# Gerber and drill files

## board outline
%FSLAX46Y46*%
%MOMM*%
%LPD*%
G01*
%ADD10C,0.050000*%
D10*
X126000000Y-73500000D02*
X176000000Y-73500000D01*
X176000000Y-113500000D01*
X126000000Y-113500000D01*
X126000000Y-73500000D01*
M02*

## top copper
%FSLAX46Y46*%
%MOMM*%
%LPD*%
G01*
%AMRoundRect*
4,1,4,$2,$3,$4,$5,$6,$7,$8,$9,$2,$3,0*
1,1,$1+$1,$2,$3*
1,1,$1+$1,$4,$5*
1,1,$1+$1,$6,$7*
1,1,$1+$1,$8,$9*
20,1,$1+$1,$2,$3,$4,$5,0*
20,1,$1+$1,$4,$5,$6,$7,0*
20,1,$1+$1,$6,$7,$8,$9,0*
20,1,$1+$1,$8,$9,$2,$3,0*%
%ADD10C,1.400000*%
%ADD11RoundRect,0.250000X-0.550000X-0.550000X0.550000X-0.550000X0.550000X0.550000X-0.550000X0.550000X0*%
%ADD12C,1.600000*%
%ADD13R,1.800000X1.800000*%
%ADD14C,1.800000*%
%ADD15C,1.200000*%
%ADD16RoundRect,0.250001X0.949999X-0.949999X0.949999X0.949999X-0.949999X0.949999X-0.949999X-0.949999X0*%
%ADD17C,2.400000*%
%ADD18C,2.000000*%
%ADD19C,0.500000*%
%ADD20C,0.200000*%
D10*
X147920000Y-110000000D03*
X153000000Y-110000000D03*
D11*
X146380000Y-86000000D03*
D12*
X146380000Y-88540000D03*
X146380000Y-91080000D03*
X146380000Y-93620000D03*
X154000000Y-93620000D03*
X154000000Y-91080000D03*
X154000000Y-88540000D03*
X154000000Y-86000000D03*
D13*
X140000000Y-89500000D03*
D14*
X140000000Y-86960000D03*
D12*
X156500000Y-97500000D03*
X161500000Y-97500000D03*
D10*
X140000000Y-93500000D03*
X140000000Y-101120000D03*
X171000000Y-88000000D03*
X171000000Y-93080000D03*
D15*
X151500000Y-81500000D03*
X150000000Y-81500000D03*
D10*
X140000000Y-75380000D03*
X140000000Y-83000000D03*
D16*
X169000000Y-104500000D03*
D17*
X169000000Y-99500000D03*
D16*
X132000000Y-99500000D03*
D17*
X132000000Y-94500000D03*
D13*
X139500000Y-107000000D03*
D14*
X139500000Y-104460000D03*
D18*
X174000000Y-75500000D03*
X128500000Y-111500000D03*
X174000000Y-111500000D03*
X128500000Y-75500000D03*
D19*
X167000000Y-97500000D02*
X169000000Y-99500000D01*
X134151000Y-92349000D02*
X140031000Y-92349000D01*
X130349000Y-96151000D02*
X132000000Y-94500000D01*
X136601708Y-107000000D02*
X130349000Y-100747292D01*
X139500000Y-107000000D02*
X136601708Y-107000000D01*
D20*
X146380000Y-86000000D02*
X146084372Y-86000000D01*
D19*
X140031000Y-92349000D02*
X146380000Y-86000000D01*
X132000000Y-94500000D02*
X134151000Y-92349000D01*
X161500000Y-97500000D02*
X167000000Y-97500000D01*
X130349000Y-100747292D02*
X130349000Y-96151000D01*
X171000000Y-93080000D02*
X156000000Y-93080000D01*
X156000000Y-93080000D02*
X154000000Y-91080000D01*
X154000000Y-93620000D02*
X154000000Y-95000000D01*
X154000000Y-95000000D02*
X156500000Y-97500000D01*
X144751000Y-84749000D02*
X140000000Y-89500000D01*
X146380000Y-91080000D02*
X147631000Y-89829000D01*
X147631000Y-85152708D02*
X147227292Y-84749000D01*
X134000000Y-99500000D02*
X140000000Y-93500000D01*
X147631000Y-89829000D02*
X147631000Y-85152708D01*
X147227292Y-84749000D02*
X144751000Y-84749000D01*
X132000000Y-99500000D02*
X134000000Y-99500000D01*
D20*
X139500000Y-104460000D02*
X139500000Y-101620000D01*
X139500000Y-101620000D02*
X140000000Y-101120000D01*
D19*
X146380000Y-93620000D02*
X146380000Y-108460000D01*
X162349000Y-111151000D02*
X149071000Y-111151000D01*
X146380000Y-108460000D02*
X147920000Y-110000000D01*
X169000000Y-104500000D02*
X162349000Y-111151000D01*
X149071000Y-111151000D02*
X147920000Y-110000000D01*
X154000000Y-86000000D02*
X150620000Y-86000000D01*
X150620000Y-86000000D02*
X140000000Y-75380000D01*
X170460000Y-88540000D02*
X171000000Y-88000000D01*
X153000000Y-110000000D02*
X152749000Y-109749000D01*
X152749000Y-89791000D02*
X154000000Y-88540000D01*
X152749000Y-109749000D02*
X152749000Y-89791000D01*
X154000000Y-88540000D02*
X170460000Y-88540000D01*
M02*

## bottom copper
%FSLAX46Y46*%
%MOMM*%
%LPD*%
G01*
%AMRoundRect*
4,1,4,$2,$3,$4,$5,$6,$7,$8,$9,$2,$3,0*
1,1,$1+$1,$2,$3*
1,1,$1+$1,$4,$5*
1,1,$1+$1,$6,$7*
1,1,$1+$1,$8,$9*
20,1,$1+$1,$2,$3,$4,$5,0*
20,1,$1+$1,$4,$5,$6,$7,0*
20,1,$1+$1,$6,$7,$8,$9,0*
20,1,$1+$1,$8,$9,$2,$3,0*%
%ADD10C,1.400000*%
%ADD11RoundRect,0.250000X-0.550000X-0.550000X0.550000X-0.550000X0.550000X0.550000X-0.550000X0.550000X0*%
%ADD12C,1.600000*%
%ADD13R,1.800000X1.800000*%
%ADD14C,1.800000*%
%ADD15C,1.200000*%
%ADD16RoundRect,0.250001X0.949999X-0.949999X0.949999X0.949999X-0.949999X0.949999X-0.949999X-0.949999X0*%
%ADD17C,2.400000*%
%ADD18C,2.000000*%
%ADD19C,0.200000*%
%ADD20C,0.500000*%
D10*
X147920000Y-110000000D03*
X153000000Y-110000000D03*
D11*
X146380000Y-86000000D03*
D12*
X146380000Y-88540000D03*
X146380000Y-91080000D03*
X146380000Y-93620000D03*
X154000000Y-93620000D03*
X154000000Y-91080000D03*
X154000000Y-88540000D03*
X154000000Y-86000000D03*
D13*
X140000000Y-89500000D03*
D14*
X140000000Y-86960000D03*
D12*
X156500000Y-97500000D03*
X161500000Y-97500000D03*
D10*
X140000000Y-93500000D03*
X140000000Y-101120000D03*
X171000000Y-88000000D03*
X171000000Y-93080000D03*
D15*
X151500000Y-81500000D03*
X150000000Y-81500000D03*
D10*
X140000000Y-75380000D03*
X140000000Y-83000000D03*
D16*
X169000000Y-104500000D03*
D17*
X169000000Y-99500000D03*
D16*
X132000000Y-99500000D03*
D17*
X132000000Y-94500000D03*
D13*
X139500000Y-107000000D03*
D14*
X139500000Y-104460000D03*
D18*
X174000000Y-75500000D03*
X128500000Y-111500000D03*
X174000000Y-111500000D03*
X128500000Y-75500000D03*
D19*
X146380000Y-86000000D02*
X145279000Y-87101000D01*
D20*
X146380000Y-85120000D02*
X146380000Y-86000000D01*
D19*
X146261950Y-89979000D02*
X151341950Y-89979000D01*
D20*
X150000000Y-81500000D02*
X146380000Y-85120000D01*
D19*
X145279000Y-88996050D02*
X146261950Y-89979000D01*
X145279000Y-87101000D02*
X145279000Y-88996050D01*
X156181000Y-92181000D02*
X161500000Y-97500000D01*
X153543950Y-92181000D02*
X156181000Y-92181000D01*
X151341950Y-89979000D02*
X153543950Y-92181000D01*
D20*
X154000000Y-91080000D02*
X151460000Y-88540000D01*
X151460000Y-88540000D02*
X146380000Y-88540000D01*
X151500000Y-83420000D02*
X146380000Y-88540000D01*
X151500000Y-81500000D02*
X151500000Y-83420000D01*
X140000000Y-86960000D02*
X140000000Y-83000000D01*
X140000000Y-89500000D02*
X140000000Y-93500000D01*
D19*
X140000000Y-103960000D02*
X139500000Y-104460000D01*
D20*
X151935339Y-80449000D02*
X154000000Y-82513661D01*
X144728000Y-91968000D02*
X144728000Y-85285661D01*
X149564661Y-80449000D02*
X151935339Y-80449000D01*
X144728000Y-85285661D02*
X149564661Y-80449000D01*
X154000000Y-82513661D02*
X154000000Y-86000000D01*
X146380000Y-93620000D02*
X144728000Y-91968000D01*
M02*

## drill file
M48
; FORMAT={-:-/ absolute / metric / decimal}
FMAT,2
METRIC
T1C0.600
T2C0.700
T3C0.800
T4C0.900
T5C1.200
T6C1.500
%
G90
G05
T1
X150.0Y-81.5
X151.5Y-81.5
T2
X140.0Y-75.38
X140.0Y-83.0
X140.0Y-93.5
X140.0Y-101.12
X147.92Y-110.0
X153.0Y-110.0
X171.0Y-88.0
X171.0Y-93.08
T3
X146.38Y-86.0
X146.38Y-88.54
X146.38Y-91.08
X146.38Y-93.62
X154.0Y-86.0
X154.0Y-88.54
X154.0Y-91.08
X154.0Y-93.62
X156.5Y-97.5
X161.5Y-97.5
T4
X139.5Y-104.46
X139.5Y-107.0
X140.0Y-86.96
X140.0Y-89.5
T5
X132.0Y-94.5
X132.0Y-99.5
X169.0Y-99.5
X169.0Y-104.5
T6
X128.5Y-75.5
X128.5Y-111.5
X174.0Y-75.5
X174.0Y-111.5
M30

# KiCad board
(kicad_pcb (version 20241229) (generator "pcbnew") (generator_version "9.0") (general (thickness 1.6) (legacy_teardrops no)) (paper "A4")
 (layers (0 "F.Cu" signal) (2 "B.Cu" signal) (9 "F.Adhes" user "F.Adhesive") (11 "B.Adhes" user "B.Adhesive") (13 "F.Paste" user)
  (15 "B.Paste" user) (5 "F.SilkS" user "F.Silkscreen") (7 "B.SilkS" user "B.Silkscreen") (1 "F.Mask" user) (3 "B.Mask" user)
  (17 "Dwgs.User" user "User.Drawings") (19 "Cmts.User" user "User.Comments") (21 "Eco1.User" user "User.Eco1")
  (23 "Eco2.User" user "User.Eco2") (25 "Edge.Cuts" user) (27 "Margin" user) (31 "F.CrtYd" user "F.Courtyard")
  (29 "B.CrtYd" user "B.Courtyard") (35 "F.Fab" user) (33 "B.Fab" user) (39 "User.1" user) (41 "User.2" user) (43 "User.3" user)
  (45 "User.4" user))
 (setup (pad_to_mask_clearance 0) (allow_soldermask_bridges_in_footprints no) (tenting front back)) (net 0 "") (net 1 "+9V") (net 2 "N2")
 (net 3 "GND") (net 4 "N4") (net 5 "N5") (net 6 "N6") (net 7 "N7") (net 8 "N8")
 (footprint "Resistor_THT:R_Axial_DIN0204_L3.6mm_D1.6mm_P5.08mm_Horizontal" (layer "F.Cu") (at 147.92 110)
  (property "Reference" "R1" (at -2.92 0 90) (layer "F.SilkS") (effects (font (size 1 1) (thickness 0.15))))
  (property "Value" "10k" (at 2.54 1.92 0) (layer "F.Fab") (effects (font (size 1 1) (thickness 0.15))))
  (pad "1" thru_hole circle (at 0 0) (size 1.4 1.4) (drill 0.7) (layers "*.Cu" "*.Mask") (remove_unused_layers no) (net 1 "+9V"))
  (pad "2" thru_hole circle (at 5.08 0) (size 1.4 1.4) (drill 0.7) (layers "*.Cu" "*.Mask") (remove_unused_layers no) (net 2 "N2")))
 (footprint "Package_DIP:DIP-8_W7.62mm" (layer "F.Cu") (at 146.38 86)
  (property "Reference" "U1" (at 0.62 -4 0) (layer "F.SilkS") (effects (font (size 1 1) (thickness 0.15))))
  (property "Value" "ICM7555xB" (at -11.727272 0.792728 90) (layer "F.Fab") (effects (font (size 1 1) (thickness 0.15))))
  (pad "1" thru_hole roundrect (at 0 0) (size 1.6 1.6) (drill 0.8) (layers "*.Cu" "*.Mask") (remove_unused_layers no)
   (roundrect_rratio 0.15625) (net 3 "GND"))
  (pad "2" thru_hole circle (at 0 2.54) (size 1.6 1.6) (drill 0.8) (layers "*.Cu" "*.Mask") (remove_unused_layers no) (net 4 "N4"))
  (pad "3" thru_hole circle (at 0 5.08) (size 1.6 1.6) (drill 0.8) (layers "*.Cu" "*.Mask") (remove_unused_layers no) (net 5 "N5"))
  (pad "4" thru_hole circle (at 0 7.62) (size 1.6 1.6) (drill 0.8) (layers "*.Cu" "*.Mask") (remove_unused_layers no) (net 1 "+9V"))
  (pad "5" thru_hole circle (at 7.62 7.62) (size 1.6 1.6) (drill 0.8) (layers "*.Cu" "*.Mask") (remove_unused_layers no) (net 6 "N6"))
  (pad "6" thru_hole circle (at 7.62 5.08) (size 1.6 1.6) (drill 0.8) (layers "*.Cu" "*.Mask") (remove_unused_layers no) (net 4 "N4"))
  (pad "7" thru_hole circle (at 7.62 2.54) (size 1.6 1.6) (drill 0.8) (layers "*.Cu" "*.Mask") (remove_unused_layers no) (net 2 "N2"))
  (pad "8" thru_hole circle (at 7.62 0) (size 1.6 1.6) (drill 0.8) (layers "*.Cu" "*.Mask") (remove_unused_layers no) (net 1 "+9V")))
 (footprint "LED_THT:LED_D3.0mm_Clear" (layer "F.Cu") (at 140 89.5 90)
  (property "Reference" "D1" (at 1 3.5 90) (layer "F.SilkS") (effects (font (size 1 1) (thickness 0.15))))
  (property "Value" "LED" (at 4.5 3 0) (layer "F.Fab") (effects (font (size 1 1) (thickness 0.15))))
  (pad "1" thru_hole rect (at 0 0 90) (size 1.8 1.8) (drill 0.9) (layers "*.Cu" "*.Mask") (remove_unused_layers no) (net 5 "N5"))
  (pad "2" thru_hole circle (at 2.54 0 90) (size 1.8 1.8) (drill 0.9) (layers "*.Cu" "*.Mask") (remove_unused_layers no) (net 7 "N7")))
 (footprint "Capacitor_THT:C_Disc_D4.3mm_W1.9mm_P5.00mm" (layer "F.Cu") (at 156.5 97.5)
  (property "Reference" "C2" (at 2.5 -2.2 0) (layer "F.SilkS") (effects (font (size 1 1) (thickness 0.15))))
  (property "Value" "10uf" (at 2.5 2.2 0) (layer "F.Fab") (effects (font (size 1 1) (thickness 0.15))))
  (pad "1" thru_hole circle (at 0 0) (size 1.6 1.6) (drill 0.8) (layers "*.Cu" "*.Mask") (remove_unused_layers no) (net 6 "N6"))
  (pad "2" thru_hole circle (at 5 0) (size 1.6 1.6) (drill 0.8) (layers "*.Cu" "*.Mask") (remove_unused_layers no) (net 3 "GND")))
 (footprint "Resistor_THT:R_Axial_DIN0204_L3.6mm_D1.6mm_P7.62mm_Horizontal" (layer "F.Cu") (at 140 93.5 -90)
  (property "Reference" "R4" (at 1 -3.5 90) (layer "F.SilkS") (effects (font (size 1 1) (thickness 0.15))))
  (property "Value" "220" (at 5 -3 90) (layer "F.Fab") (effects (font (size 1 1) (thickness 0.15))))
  (pad "1" thru_hole circle (at 0 0 270) (size 1.4 1.4) (drill 0.7) (layers "*.Cu" "*.Mask") (remove_unused_layers no) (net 5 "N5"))
  (pad "2" thru_hole circle (at 7.62 0 270) (size 1.4 1.4) (drill 0.7) (layers "*.Cu" "*.Mask") (remove_unused_layers no) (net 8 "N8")))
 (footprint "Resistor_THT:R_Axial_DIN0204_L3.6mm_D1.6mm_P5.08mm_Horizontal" (layer "F.Cu") (at 171 88 -90)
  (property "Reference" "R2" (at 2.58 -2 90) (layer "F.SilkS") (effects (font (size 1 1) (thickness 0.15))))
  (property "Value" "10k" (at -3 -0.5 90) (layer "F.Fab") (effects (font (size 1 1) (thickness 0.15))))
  (pad "1" thru_hole circle (at 0 0 270) (size 1.4 1.4) (drill 0.7) (layers "*.Cu" "*.Mask") (remove_unused_layers no) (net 2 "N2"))
  (pad "2" thru_hole circle (at 5.08 0 270) (size 1.4 1.4) (drill 0.7) (layers "*.Cu" "*.Mask") (remove_unused_layers no) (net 4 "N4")))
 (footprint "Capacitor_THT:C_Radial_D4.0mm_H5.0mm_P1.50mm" (layer "F.Cu") (at 151.5 81.5 180)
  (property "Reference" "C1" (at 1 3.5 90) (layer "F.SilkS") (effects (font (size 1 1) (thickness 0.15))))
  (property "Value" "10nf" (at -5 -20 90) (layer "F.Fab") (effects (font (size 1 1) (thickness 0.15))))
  (pad "1" thru_hole circle (at 0 0 180) (size 1.2 1.2) (drill 0.6) (layers "*.Cu" "*.Mask") (remove_unused_layers no) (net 4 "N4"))
  (pad "2" thru_hole circle (at 1.5 0 180) (size 1.2 1.2) (drill 0.6) (layers "*.Cu" "*.Mask") (remove_unused_layers no) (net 3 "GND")))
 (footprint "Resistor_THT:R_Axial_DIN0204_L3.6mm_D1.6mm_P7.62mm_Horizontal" (layer "F.Cu") (at 140 75.38 -90)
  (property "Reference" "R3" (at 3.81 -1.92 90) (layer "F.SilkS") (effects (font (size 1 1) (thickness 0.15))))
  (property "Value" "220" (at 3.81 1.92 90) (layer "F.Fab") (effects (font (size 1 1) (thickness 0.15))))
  (pad "1" thru_hole circle (at 0 0 270) (size 1.4 1.4) (drill 0.7) (layers "*.Cu" "*.Mask") (remove_unused_layers no) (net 1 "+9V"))
  (pad "2" thru_hole circle (at 7.62 0 270) (size 1.4 1.4) (drill 0.7) (layers "*.Cu" "*.Mask") (remove_unused_layers no) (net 7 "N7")))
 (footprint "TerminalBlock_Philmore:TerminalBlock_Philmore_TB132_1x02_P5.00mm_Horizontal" (layer "F.Cu") (at 169 104.5 90)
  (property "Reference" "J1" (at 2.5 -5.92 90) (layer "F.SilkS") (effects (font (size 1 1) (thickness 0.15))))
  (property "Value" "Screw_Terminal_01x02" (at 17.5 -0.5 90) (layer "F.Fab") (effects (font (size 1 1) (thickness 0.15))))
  (pad "1" thru_hole roundrect (at 0 0 90) (size 2.4 2.4) (drill 1.2) (layers "*.Cu" "*.Mask") (remove_unused_layers no)
   (roundrect_rratio 0.104167) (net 1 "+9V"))
  (pad "2" thru_hole circle (at 5 0 90) (size 2.4 2.4) (drill 1.2) (layers "*.Cu" "*.Mask") (remove_unused_layers no) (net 3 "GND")))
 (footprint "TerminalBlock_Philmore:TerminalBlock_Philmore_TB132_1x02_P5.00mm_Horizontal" (layer "F.Cu") (at 132 99.5 90)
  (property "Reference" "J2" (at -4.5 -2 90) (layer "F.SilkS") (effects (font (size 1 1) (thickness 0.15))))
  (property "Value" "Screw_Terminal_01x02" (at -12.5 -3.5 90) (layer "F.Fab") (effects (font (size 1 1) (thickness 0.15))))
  (pad "1" thru_hole roundrect (at 0 0 90) (size 2.4 2.4) (drill 1.2) (layers "*.Cu" "*.Mask") (remove_unused_layers no)
   (roundrect_rratio 0.104167) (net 5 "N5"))
  (pad "2" thru_hole circle (at 5 0 90) (size 2.4 2.4) (drill 1.2) (layers "*.Cu" "*.Mask") (remove_unused_layers no) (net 3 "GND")))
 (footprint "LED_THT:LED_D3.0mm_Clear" (layer "F.Cu") (at 139.5 107 90)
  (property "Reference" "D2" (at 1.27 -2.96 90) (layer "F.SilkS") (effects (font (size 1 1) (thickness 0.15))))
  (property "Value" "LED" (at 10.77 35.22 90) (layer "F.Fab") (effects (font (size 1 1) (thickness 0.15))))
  (pad "1" thru_hole rect (at 0 0 90) (size 1.8 1.8) (drill 0.9) (layers "*.Cu" "*.Mask") (remove_unused_layers no) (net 3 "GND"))
  (pad "2" thru_hole circle (at 2.54 0 90) (size 1.8 1.8) (drill 0.9) (layers "*.Cu" "*.Mask") (remove_unused_layers no) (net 8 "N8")))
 (gr_rect (start 126 73.5) (end 176 113.5) (stroke (width 0.05) (type default)) (fill no) (layer "Edge.Cuts"))
 (via (at 174 75.5) (size 2) (drill 1.5) (layers "F.Cu" "B.Cu") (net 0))
 (via (at 128.5 111.5) (size 2) (drill 1.5) (layers "F.Cu" "B.Cu") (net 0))
 (via (at 174 111.5) (size 2) (drill 1.5) (layers "F.Cu" "B.Cu") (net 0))
 (via (at 128.5 75.5) (size 2) (drill 1.5) (layers "F.Cu" "B.Cu") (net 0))
 (segment (start 167 97.5) (end 169 99.5) (width 0.5) (layer "F.Cu") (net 3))
 (segment (start 134.151 92.349) (end 140.031 92.349) (width 0.5) (layer "F.Cu") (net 3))
 (segment (start 130.349 96.151) (end 132 94.5) (width 0.5) (layer "F.Cu") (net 3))
 (segment (start 136.601708 107) (end 130.349 100.747292) (width 0.5) (layer "F.Cu") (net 3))
 (segment (start 139.5 107) (end 136.601708 107) (width 0.5) (layer "F.Cu") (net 3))
 (segment (start 146.38 86) (end 146.084372 86) (width 0.2) (layer "F.Cu") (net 3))
 (segment (start 140.031 92.349) (end 146.38 86) (width 0.5) (layer "F.Cu") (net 3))
 (segment (start 132 94.5) (end 134.151 92.349) (width 0.5) (layer "F.Cu") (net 3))
 (segment (start 161.5 97.5) (end 167 97.5) (width 0.5) (layer "F.Cu") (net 3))
 (segment (start 130.349 100.747292) (end 130.349 96.151) (width 0.5) (layer "F.Cu") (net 3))
 (segment (start 146.38 86) (end 145.279 87.101) (width 0.2) (layer "B.Cu") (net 3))
 (segment (start 146.38 85.12) (end 146.38 86) (width 0.5) (layer "B.Cu") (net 3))
 (segment (start 146.26195 89.979) (end 151.34195 89.979) (width 0.2) (layer "B.Cu") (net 3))
 (segment (start 150 81.5) (end 146.38 85.12) (width 0.5) (layer "B.Cu") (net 3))
 (segment (start 145.279 88.99605) (end 146.26195 89.979) (width 0.2) (layer "B.Cu") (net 3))
 (segment (start 145.279 87.101) (end 145.279 88.99605) (width 0.2) (layer "B.Cu") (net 3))
 (segment (start 156.181 92.181) (end 161.5 97.5) (width 0.2) (layer "B.Cu") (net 3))
 (segment (start 153.54395 92.181) (end 156.181 92.181) (width 0.2) (layer "B.Cu") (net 3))
 (segment (start 151.34195 89.979) (end 153.54395 92.181) (width 0.2) (layer "B.Cu") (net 3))
 (segment (start 171 93.08) (end 156 93.08) (width 0.5) (layer "F.Cu") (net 4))
 (segment (start 156 93.08) (end 154 91.08) (width 0.5) (layer "F.Cu") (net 4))
 (segment (start 154 91.08) (end 151.46 88.54) (width 0.5) (layer "B.Cu") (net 4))
 (segment (start 151.46 88.54) (end 146.38 88.54) (width 0.5) (layer "B.Cu") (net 4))
 (segment (start 151.5 83.42) (end 146.38 88.54) (width 0.5) (layer "B.Cu") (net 4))
 (segment (start 151.5 81.5) (end 151.5 83.42) (width 0.5) (layer "B.Cu") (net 4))
 (segment (start 154 93.62) (end 154 95) (width 0.5) (layer "F.Cu") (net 6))
 (segment (start 154 95) (end 156.5 97.5) (width 0.5) (layer "F.Cu") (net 6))
 (segment (start 140 86.96) (end 140 83) (width 0.5) (layer "B.Cu") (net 7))
 (segment (start 144.751 84.749) (end 140 89.5) (width 0.5) (layer "F.Cu") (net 5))
 (segment (start 146.38 91.08) (end 147.631 89.829) (width 0.5) (layer "F.Cu") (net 5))
 (segment (start 147.631 85.152708) (end 147.227292 84.749) (width 0.5) (layer "F.Cu") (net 5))
 (segment (start 134 99.5) (end 140 93.5) (width 0.5) (layer "F.Cu") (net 5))
 (segment (start 147.631 89.829) (end 147.631 85.152708) (width 0.5) (layer "F.Cu") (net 5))
 (segment (start 147.227292 84.749) (end 144.751 84.749) (width 0.5) (layer "F.Cu") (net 5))
 (segment (start 132 99.5) (end 134 99.5) (width 0.5) (layer "F.Cu") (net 5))
 (segment (start 140 89.5) (end 140 93.5) (width 0.5) (layer "B.Cu") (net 5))
 (segment (start 139.5 104.46) (end 139.5 101.62) (width 0.2) (layer "F.Cu") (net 8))
 (segment (start 139.5 101.62) (end 140 101.12) (width 0.2) (layer "F.Cu") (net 8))
 (segment (start 140 103.96) (end 139.5 104.46) (width 0.2) (layer "B.Cu") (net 8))
 (segment (start 146.38 93.62) (end 146.38 108.46) (width 0.5) (layer "F.Cu") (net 1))
 (segment (start 162.349 111.151) (end 149.071 111.151) (width 0.5) (layer "F.Cu") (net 1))
 (segment (start 146.38 108.46) (end 147.92 110) (width 0.5) (layer "F.Cu") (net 1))
 (segment (start 169 104.5) (end 162.349 111.151) (width 0.5) (layer "F.Cu") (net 1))
 (segment (start 149.071 111.151) (end 147.92 110) (width 0.5) (layer "F.Cu") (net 1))
 (segment (start 154 86) (end 150.62 86) (width 0.5) (layer "F.Cu") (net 1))
 (segment (start 150.62 86) (end 140 75.38) (width 0.5) (layer "F.Cu") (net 1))
 (segment (start 151.935339 80.449) (end 154 82.513661) (width 0.5) (layer "B.Cu") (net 1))
 (segment (start 144.728 91.968) (end 144.728 85.285661) (width 0.5) (layer "B.Cu") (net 1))
 (segment (start 149.564661 80.449) (end 151.935339 80.449) (width 0.5) (layer "B.Cu") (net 1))
 (segment (start 144.728 85.285661) (end 149.564661 80.449) (width 0.5) (layer "B.Cu") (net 1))
 (segment (start 154 82.513661) (end 154 86) (width 0.5) (layer "B.Cu") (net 1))
 (segment (start 146.38 93.62) (end 144.728 91.968) (width 0.5) (layer "B.Cu") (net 1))
 (segment (start 170.46 88.54) (end 171 88) (width 0.5) (layer "F.Cu") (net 2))
 (segment (start 153 110) (end 152.749 109.749) (width 0.5) (layer "F.Cu") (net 2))
 (segment (start 152.749 89.791) (end 154 88.54) (width 0.5) (layer "F.Cu") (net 2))
 (segment (start 152.749 109.749) (end 152.749 89.791) (width 0.5) (layer "F.Cu") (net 2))
 (segment (start 154 88.54) (end 170.46 88.54) (width 0.5) (layer "F.Cu") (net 2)))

